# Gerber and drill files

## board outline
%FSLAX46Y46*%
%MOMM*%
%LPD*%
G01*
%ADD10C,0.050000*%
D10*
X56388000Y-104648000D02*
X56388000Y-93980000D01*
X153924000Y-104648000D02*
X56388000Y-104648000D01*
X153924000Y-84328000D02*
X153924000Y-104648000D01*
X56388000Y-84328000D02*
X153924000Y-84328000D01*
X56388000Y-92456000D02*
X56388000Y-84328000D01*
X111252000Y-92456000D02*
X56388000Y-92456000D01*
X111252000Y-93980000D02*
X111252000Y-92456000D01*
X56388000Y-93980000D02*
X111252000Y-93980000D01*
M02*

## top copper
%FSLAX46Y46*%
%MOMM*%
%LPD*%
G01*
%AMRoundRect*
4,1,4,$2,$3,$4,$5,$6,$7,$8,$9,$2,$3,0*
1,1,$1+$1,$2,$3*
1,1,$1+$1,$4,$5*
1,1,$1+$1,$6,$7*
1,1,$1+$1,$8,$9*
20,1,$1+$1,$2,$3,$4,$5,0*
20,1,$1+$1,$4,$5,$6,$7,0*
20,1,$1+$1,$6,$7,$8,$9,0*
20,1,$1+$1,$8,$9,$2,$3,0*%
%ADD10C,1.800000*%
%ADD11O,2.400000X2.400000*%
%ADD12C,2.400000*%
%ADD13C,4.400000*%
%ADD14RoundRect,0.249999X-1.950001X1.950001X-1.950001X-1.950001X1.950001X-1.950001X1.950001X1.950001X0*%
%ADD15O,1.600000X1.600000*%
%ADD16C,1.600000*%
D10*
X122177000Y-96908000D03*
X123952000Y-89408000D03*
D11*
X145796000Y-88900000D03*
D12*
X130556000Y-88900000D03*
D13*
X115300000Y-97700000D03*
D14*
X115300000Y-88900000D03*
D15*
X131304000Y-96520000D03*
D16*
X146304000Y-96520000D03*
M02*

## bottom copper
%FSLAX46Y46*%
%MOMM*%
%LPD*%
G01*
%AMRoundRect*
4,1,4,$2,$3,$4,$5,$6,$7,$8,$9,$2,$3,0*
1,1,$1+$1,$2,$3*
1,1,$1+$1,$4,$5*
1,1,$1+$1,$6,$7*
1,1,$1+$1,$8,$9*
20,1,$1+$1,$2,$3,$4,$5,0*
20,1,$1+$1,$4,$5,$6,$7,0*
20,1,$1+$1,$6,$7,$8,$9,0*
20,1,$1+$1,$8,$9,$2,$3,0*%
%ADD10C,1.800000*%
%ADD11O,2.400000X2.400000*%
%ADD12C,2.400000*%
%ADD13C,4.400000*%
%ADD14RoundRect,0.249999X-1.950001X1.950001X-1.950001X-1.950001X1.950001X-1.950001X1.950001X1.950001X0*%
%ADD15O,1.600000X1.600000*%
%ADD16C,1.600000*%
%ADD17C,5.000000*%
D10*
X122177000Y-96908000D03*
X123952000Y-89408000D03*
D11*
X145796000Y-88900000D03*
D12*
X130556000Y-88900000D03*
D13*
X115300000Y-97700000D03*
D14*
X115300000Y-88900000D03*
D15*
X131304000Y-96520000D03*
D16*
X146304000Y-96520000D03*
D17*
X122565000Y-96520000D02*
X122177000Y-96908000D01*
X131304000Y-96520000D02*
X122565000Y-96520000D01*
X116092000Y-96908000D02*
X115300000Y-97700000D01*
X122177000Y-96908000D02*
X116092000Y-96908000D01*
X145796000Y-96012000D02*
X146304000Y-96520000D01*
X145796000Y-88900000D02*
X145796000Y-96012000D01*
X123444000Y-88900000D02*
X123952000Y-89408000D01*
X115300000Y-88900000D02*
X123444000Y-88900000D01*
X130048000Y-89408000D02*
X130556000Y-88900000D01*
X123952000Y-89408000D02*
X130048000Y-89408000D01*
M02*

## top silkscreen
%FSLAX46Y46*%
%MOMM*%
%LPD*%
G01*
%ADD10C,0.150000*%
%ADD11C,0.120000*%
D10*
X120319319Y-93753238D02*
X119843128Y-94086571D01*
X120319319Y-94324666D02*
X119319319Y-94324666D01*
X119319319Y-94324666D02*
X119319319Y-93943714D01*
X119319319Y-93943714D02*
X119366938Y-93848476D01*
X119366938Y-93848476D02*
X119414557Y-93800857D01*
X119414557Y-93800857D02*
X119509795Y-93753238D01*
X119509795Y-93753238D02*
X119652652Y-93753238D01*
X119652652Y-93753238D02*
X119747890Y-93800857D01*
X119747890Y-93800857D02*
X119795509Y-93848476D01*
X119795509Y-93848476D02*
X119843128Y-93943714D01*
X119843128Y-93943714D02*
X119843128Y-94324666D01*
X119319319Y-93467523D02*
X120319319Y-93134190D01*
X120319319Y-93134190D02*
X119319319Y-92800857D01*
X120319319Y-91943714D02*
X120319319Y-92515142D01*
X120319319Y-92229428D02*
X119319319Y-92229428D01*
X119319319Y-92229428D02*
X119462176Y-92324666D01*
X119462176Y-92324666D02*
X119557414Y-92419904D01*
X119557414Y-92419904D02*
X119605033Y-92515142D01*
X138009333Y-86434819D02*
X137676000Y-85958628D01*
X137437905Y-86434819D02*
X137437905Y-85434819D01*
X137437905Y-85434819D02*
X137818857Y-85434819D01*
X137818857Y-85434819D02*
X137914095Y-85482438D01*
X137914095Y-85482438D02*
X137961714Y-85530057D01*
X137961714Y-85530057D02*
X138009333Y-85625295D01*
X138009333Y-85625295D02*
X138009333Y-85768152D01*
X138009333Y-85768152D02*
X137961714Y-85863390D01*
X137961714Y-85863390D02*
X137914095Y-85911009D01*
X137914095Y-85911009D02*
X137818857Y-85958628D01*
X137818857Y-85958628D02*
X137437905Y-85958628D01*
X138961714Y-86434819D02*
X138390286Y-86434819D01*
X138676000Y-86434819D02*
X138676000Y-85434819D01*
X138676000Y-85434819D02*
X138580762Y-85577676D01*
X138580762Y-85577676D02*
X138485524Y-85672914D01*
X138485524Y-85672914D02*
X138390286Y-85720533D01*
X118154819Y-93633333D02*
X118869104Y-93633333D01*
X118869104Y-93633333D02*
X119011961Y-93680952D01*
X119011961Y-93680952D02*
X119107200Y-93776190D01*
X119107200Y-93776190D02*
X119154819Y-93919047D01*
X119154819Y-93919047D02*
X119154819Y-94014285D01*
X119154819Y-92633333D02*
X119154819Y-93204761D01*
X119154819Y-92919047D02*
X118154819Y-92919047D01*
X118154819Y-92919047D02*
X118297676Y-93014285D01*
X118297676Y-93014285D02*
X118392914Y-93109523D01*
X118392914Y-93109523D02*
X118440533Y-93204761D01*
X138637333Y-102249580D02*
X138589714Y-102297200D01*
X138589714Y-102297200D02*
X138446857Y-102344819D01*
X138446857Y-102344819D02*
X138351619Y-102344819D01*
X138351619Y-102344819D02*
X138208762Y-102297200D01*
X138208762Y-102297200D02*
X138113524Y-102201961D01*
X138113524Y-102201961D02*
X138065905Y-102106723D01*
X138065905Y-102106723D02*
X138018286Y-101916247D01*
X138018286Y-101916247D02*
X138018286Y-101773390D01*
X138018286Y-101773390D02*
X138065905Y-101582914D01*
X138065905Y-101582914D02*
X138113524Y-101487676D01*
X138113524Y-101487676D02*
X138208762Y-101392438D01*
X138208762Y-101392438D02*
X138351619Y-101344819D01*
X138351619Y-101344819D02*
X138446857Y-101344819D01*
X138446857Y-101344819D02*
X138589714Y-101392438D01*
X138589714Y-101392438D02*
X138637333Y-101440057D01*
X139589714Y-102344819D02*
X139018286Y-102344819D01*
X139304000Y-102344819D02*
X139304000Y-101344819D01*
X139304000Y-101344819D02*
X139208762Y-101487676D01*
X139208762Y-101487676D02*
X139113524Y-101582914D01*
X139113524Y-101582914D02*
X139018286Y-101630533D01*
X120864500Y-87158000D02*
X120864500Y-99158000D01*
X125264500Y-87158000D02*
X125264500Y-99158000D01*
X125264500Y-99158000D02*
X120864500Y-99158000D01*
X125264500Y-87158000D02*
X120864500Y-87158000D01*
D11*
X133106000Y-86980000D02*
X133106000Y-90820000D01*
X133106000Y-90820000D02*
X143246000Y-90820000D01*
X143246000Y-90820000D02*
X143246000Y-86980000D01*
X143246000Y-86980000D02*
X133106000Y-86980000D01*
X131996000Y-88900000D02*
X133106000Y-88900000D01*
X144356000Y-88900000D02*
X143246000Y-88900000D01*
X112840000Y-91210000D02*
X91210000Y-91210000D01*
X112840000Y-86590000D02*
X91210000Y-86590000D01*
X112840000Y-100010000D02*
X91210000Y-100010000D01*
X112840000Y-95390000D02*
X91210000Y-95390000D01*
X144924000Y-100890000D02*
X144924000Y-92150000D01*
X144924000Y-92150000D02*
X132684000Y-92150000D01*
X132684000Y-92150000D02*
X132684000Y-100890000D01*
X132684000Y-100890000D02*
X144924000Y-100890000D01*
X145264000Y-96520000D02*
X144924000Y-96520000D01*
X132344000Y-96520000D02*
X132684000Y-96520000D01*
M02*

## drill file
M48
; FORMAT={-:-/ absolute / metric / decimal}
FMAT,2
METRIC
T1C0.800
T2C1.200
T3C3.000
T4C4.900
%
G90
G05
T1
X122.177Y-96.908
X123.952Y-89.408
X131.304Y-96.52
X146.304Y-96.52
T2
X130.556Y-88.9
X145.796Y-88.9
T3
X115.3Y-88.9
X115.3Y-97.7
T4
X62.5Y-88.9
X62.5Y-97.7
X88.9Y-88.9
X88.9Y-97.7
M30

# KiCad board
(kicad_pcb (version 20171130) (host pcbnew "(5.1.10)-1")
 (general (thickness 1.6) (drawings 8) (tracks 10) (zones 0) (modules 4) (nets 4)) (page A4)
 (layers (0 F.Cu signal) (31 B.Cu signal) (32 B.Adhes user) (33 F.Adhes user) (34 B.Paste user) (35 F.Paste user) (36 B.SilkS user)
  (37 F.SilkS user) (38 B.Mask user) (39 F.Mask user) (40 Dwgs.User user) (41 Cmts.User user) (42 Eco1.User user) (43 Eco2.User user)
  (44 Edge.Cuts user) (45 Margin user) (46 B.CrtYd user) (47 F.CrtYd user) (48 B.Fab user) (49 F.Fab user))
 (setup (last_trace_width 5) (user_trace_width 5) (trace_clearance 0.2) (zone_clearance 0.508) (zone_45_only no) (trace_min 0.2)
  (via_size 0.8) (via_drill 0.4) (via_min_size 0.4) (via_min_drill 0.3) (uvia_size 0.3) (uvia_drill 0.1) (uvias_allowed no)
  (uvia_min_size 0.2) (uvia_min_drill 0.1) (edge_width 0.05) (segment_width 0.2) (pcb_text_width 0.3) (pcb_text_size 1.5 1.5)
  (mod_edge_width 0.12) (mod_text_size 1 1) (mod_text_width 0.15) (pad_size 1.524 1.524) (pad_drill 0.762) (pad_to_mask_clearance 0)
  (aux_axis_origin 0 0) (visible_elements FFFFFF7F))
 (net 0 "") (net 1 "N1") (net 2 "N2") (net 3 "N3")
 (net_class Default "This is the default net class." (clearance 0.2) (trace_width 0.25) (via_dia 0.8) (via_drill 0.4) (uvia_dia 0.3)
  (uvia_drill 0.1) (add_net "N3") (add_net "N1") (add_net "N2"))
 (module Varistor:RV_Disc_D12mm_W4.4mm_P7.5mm (layer F.Cu) (at 123.952 89.408 270)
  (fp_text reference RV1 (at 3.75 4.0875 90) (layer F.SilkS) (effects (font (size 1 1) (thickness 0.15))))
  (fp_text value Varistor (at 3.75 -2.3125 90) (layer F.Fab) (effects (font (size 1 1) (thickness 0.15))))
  (fp_line (start -2.25 3.0875) (end 9.75 3.0875) (layer F.SilkS) (width 0.15))
  (fp_line (start -2.25 -1.3125) (end 9.75 -1.3125) (layer F.SilkS) (width 0.15))
  (fp_line (start 9.75 -1.3125) (end 9.75 3.0875) (layer F.SilkS) (width 0.15))
  (fp_line (start -2.25 -1.3125) (end -2.25 3.0875) (layer F.SilkS) (width 0.15))
  (pad 2 thru_hole circle (at 7.5 1.775 270) (size 1.8 1.8) (drill 0.8) (layers *.Cu *.Mask) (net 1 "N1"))
  (pad 1 thru_hole circle (at 0 0 270) (size 1.8 1.8) (drill 0.8) (layers *.Cu *.Mask) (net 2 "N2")))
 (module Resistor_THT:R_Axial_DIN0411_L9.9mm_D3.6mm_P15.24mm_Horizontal (layer F.Cu) (at 130.556 88.9)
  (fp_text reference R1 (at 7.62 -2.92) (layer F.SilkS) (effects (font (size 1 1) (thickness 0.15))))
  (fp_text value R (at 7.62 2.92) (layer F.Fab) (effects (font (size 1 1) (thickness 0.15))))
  (fp_line (start 2.55 -1.92) (end 2.55 1.92) (layer F.SilkS) (width 0.12))
  (fp_line (start 2.55 1.92) (end 12.69 1.92) (layer F.SilkS) (width 0.12))
  (fp_line (start 12.69 1.92) (end 12.69 -1.92) (layer F.SilkS) (width 0.12))
  (fp_line (start 12.69 -1.92) (end 2.55 -1.92) (layer F.SilkS) (width 0.12))
  (fp_line (start 1.44 0) (end 2.55 0) (layer F.SilkS) (width 0.12))
  (fp_line (start 13.8 0) (end 12.69 0) (layer F.SilkS) (width 0.12))
  (pad 2 thru_hole oval (at 15.24 0) (size 2.4 2.4) (drill 1.2) (layers *.Cu *.Mask) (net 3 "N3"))
  (pad 1 thru_hole circle (at 0 0) (size 2.4 2.4) (drill 1.2) (layers *.Cu *.Mask) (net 2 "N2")))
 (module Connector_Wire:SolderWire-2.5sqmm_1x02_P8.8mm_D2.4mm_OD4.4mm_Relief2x (layer F.Cu) (at 115.3 88.9 270)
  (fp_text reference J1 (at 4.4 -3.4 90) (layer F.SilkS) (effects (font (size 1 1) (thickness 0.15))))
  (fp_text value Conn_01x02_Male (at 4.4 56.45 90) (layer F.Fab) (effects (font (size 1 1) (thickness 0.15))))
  (fp_line (start 2.31 2.46) (end 2.31 24.09) (layer F.SilkS) (width 0.12))
  (fp_line (start -2.31 2.46) (end -2.31 24.09) (layer F.SilkS) (width 0.12))
  (fp_line (start 11.11 2.46) (end 11.11 24.09) (layer F.SilkS) (width 0.12))
  (fp_line (start 6.49 2.46) (end 6.49 24.09) (layer F.SilkS) (width 0.12))
  (pad "" np_thru_hole circle (at 8.8 52.8 270) (size 4.9 4.9) (drill 4.9) (layers *.Cu *.Mask))
  (pad "" np_thru_hole circle (at 8.8 26.4 270) (size 4.9 4.9) (drill 4.9) (layers *.Cu *.Mask))
  (pad "" np_thru_hole circle (at 0 52.8 270) (size 4.9 4.9) (drill 4.9) (layers *.Cu *.Mask))
  (pad "" np_thru_hole circle (at 0 26.4 270) (size 4.9 4.9) (drill 4.9) (layers *.Cu *.Mask))
  (pad 2 thru_hole circle (at 8.8 0 270) (size 4.4 4.4) (drill 3) (layers *.Cu *.Mask) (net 1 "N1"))
  (pad 1 thru_hole roundrect (at 0 0 270) (size 4.4 4.4) (drill 3) (layers *.Cu *.Mask) (roundrect_rratio 0.056818) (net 2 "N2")))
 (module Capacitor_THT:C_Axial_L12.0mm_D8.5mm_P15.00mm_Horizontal (layer F.Cu) (at 146.304 96.52 180)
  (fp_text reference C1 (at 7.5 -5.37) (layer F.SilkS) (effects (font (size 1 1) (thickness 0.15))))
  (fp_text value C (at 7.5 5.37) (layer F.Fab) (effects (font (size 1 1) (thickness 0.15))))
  (fp_line (start 1.38 -4.37) (end 1.38 4.37) (layer F.SilkS) (width 0.12))
  (fp_line (start 1.38 4.37) (end 13.62 4.37) (layer F.SilkS) (width 0.12))
  (fp_line (start 13.62 4.37) (end 13.62 -4.37) (layer F.SilkS) (width 0.12))
  (fp_line (start 13.62 -4.37) (end 1.38 -4.37) (layer F.SilkS) (width 0.12))
  (fp_line (start 1.04 0) (end 1.38 0) (layer F.SilkS) (width 0.12))
  (fp_line (start 13.96 0) (end 13.62 0) (layer F.SilkS) (width 0.12))
  (pad 2 thru_hole oval (at 15 0 180) (size 1.6 1.6) (drill 0.8) (layers *.Cu *.Mask) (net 1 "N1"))
  (pad 1 thru_hole circle (at 0 0 180) (size 1.6 1.6) (drill 0.8) (layers *.Cu *.Mask) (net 3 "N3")))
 (gr_line (start 56.388 104.648) (end 56.388 93.98) (layer Edge.Cuts) (width 0.05))
 (gr_line (start 153.924 104.648) (end 56.388 104.648) (layer Edge.Cuts) (width 0.05))
 (gr_line (start 153.924 84.328) (end 153.924 104.648) (layer Edge.Cuts) (width 0.05))
 (gr_line (start 56.388 84.328) (end 153.924 84.328) (layer Edge.Cuts) (width 0.05))
 (gr_line (start 56.388 92.456) (end 56.388 84.328) (layer Edge.Cuts) (width 0.05))
 (gr_line (start 111.252 92.456) (end 56.388 92.456) (layer Edge.Cuts) (width 0.05))
 (gr_line (start 111.252 93.98) (end 111.252 92.456) (layer Edge.Cuts) (width 0.05))
 (gr_line (start 56.388 93.98) (end 111.252 93.98) (layer Edge.Cuts) (width 0.05))
 (segment (start 122.565 96.52) (end 122.177 96.908) (width 5) (layer B.Cu) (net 1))
 (segment (start 131.304 96.52) (end 122.565 96.52) (width 5) (layer B.Cu) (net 1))
 (segment (start 116.092 96.908) (end 115.3 97.7) (width 5) (layer B.Cu) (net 1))
 (segment (start 122.177 96.908) (end 116.092 96.908) (width 5) (layer B.Cu) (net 1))
 (segment (start 145.796 96.012) (end 146.304 96.52) (width 5) (layer B.Cu) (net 3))
 (segment (start 145.796 88.9) (end 145.796 96.012) (width 5) (layer B.Cu) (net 3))
 (segment (start 123.444 88.9) (end 123.952 89.408) (width 5) (layer B.Cu) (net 2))
 (segment (start 115.3 88.9) (end 123.444 88.9) (width 5) (layer B.Cu) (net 2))
 (segment (start 130.048 89.408) (end 130.556 88.9) (width 5) (layer B.Cu) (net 2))
 (segment (start 123.952 89.408) (end 130.048 89.408) (width 5) (layer B.Cu) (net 2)))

